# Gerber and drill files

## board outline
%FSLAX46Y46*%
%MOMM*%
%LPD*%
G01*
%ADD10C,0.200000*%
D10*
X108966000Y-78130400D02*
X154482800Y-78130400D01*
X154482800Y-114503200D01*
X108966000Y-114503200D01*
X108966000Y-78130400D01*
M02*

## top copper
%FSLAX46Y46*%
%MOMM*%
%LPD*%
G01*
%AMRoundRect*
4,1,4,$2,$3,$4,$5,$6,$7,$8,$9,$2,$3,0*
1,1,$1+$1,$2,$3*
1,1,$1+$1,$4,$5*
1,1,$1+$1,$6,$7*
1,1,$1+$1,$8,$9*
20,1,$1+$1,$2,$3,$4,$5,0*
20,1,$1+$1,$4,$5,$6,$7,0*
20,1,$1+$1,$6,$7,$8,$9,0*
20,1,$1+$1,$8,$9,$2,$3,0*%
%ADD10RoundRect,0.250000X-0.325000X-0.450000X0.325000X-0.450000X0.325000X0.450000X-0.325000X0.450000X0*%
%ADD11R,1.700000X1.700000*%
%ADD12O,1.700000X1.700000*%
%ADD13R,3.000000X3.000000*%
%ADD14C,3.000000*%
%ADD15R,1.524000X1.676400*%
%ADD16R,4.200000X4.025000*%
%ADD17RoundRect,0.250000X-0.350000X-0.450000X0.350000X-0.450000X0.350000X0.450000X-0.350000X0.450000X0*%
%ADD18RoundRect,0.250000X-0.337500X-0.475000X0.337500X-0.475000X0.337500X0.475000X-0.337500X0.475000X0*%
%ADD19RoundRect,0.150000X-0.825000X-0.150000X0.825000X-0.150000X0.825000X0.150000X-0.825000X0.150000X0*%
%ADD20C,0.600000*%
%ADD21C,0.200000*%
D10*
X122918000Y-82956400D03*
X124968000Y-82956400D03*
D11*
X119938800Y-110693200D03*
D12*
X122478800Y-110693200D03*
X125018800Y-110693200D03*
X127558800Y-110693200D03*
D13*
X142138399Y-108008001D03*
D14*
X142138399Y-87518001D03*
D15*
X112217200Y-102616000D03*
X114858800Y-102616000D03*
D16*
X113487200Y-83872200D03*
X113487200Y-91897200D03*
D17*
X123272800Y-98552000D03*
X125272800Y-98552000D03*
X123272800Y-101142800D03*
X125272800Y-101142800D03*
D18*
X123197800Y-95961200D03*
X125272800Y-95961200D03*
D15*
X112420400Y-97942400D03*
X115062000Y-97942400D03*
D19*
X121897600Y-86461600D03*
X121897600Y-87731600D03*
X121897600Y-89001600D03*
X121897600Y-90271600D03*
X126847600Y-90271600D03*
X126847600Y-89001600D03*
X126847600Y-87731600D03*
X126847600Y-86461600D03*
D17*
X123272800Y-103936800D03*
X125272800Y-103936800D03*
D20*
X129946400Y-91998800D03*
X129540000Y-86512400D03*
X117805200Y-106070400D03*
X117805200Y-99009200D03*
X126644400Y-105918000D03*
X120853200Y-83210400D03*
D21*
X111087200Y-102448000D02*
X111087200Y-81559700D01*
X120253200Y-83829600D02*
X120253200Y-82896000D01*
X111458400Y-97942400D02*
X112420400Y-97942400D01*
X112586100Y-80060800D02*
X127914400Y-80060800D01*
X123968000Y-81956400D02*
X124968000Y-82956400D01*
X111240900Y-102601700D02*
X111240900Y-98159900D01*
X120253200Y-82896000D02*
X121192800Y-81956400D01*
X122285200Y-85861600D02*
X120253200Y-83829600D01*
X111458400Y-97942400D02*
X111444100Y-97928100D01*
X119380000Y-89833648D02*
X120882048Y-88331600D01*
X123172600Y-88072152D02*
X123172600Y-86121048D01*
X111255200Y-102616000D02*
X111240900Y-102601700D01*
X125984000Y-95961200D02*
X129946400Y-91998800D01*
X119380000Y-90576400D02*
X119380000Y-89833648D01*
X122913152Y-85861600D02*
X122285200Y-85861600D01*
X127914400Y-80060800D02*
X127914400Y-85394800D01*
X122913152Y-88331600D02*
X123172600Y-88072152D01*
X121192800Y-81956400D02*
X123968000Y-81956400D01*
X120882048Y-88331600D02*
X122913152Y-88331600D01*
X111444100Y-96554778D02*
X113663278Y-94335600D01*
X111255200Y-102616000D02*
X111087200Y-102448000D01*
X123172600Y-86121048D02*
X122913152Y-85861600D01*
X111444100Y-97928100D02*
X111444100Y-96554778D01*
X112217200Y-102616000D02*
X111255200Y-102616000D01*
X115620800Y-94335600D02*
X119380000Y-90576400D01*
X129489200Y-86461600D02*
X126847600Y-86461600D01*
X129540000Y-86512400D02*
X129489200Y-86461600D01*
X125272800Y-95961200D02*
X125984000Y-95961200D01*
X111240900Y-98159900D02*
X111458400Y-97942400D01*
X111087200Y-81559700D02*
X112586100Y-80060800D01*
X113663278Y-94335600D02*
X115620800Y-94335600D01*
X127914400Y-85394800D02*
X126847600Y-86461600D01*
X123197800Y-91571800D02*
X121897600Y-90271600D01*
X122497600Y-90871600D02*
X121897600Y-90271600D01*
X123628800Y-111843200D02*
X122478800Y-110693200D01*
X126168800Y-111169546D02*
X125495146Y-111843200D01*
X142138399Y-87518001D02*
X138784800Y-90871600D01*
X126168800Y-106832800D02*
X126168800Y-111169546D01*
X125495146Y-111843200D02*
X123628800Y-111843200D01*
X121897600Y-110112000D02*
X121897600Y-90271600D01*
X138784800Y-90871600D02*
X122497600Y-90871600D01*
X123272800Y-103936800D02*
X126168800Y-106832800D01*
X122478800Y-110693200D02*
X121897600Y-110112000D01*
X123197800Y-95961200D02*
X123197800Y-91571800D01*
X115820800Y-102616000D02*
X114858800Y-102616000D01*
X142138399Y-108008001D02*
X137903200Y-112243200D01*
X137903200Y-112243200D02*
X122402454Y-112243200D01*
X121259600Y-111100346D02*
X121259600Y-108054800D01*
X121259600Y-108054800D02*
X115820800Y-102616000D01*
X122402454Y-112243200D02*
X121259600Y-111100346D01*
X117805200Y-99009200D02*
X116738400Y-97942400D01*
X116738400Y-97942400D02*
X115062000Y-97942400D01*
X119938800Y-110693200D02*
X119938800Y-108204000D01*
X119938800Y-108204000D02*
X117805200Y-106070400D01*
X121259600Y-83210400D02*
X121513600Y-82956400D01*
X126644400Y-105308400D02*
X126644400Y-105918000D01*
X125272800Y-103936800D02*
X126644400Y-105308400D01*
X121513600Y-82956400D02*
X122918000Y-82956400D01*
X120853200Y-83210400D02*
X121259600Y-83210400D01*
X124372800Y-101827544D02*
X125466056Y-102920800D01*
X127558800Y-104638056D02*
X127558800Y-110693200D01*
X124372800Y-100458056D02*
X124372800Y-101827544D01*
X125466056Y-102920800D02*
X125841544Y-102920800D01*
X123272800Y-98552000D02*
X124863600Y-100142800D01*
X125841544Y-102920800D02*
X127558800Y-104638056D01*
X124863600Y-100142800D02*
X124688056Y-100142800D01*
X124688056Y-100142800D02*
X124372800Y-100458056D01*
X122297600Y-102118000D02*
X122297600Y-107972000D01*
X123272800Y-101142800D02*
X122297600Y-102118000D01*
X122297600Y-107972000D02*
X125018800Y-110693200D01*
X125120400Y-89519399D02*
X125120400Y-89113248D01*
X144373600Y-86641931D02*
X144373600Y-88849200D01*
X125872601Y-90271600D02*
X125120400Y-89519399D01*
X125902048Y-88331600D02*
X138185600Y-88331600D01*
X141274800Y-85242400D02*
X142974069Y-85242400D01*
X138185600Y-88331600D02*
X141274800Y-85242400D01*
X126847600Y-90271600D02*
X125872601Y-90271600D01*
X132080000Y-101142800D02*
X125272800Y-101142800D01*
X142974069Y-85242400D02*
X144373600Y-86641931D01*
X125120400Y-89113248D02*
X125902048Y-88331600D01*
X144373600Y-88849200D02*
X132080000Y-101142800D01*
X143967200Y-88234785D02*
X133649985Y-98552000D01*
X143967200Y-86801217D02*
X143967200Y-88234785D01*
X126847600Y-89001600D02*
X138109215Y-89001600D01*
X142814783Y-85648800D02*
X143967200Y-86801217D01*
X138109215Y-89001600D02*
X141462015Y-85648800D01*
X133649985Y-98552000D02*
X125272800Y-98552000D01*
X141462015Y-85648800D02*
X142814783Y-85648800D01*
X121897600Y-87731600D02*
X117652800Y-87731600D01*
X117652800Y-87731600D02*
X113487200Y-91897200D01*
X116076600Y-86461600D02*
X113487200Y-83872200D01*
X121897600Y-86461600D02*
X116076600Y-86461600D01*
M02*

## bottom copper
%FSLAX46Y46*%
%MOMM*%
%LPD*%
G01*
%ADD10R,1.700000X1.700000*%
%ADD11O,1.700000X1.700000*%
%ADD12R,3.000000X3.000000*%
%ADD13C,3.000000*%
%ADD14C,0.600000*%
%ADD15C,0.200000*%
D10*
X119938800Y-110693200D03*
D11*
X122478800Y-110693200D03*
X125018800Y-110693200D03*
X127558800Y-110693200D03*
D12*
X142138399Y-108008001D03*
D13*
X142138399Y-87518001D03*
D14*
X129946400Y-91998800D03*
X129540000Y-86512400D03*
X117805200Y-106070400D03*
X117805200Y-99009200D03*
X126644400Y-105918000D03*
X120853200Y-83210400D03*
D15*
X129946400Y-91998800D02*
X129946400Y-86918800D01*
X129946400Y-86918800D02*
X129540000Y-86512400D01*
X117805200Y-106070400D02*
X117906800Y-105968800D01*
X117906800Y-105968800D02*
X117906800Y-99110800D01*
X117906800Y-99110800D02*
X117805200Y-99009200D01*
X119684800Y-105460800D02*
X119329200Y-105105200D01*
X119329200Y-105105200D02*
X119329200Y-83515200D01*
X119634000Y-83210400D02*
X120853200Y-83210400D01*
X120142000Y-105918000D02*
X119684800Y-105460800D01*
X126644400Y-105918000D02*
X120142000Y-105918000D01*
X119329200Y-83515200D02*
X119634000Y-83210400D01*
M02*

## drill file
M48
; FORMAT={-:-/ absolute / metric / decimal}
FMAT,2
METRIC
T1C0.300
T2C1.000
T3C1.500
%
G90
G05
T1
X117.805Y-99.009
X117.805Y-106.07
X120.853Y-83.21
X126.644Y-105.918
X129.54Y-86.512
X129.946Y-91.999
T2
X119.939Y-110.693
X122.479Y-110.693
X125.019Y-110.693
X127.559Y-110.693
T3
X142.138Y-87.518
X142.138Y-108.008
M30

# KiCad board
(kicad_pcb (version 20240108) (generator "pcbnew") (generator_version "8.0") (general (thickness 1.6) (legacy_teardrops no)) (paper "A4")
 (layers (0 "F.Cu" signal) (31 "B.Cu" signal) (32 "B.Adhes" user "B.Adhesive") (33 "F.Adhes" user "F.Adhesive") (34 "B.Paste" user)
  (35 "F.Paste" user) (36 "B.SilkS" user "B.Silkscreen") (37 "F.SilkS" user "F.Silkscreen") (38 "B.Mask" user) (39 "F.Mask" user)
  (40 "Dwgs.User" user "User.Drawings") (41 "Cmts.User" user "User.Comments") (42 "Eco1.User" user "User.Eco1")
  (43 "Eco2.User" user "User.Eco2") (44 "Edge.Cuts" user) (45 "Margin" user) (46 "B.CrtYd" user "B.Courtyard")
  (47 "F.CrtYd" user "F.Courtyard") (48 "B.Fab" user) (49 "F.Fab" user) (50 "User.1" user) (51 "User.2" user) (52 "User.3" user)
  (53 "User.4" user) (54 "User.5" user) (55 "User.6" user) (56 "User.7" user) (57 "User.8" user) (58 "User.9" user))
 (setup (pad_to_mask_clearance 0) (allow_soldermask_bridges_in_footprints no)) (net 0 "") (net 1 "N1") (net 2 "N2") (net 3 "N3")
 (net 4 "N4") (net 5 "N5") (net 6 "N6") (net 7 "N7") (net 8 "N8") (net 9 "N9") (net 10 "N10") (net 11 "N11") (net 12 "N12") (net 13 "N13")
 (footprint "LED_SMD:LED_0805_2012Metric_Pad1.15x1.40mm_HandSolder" (layer "F.Cu") (at 123.943 82.9564)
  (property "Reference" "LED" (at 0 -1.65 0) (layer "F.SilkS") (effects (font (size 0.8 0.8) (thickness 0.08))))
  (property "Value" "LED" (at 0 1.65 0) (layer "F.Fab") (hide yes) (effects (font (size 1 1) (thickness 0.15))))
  (pad "1" smd roundrect (at -1.025 0) (size 1.15 1.4) (layers "F.Cu" "F.Paste" "F.Mask") (roundrect_rratio 0.217391) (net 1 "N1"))
  (pad "2" smd roundrect (at 1.025 0) (size 1.15 1.4) (layers "F.Cu" "F.Paste" "F.Mask") (roundrect_rratio 0.217391) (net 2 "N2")))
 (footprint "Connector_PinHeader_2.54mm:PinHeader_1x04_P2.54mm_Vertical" (layer "F.Cu") (at 119.9388 110.6932 90)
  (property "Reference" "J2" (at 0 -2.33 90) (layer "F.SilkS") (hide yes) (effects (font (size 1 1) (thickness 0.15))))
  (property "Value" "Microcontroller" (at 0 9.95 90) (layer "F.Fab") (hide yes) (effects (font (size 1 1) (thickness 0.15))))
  (pad "1" thru_hole rect (at 0 0 90) (size 1.7 1.7) (drill 1) (layers "*.Cu" "*.Mask") (remove_unused_layers no) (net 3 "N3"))
  (pad "2" thru_hole oval (at 0 2.54 90) (size 1.7 1.7) (drill 1) (layers "*.Cu" "*.Mask") (remove_unused_layers no) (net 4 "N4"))
  (pad "3" thru_hole oval (at 0 5.08 90) (size 1.7 1.7) (drill 1) (layers "*.Cu" "*.Mask") (remove_unused_layers no) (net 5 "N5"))
  (pad "4" thru_hole oval (at 0 7.62 90) (size 1.7 1.7) (drill 1) (layers "*.Cu" "*.Mask") (remove_unused_layers no) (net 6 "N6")))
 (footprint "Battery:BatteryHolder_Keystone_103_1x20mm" (layer "F.Cu") (at 142.138399 108.008001 90)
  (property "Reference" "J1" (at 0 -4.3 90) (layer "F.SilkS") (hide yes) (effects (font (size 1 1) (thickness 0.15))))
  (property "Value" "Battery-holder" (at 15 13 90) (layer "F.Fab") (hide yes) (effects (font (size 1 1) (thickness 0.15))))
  (pad "1" thru_hole rect (at 0 0 90) (size 3 3) (drill 1.5) (layers "*.Cu" "*.Mask") (remove_unused_layers no) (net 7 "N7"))
  (pad "2" thru_hole circle (at 20.49 0 90) (size 3 3) (drill 1.5) (layers "*.Cu" "*.Mask") (remove_unused_layers no) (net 4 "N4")))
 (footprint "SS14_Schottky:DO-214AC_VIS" (layer "F.Cu") (at 113.538 102.616)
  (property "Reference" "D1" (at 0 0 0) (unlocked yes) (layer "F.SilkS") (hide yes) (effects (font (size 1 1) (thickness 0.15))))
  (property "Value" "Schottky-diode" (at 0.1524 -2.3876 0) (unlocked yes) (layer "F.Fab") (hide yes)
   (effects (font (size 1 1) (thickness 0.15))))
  (pad "1" smd rect (at -1.3208 0) (size 1.524 1.6764) (layers "F.Cu" "F.Paste" "F.Mask") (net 2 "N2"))
  (pad "2" smd rect (at 1.3208 0) (size 1.524 1.6764) (layers "F.Cu" "F.Paste" "F.Mask") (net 7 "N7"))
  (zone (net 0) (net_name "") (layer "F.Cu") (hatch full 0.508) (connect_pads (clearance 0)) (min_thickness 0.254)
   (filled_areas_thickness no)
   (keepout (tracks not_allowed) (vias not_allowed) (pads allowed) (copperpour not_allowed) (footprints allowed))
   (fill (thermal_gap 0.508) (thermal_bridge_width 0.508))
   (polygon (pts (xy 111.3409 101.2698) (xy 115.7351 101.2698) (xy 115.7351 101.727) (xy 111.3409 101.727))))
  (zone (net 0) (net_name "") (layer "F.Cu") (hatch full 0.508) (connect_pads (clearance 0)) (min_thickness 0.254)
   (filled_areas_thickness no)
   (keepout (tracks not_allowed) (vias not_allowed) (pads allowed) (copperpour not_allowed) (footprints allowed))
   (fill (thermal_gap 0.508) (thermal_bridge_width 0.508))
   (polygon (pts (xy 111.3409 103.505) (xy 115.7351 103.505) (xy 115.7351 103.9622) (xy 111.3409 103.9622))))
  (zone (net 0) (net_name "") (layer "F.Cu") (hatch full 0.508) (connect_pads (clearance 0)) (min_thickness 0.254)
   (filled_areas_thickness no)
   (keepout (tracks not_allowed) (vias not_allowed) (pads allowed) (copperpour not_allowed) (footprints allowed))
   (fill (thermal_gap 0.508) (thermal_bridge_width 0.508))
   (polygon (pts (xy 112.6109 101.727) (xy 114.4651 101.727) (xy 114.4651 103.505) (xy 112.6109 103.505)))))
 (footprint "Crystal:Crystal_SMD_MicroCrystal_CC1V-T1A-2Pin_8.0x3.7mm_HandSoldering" (layer "F.Cu") (at 113.4872 87.8847 -90)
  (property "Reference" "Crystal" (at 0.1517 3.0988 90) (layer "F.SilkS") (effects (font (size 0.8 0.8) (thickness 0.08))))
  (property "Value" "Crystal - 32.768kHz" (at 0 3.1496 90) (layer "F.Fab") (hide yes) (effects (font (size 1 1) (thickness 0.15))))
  (pad "1" smd rect (at -4.0125 0 270) (size 4.025 4.2) (layers "F.Cu" "F.Paste" "F.Mask") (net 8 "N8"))
  (pad "2" smd rect (at 4.0125 0 270) (size 4.025 4.2) (layers "F.Cu" "F.Paste" "F.Mask") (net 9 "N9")))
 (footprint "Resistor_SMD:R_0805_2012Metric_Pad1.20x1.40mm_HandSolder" (layer "F.Cu") (at 124.2728 98.552)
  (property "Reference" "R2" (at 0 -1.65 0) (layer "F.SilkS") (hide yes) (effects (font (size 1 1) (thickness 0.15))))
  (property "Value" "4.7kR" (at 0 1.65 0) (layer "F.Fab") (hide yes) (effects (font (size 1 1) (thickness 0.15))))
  (pad "1" smd roundrect (at -1 0) (size 1.2 1.4) (layers "F.Cu" "F.Paste" "F.Mask") (roundrect_rratio 0.208333) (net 6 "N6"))
  (pad "2" smd roundrect (at 1 0) (size 1.2 1.4) (layers "F.Cu" "F.Paste" "F.Mask") (roundrect_rratio 0.208333) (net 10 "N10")))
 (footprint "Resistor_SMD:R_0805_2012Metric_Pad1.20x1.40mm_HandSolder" (layer "F.Cu") (at 124.2728 101.1428)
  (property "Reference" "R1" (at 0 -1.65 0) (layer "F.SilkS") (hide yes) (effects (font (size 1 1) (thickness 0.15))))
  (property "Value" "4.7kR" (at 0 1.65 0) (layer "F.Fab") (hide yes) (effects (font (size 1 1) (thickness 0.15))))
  (pad "1" smd roundrect (at -1 0) (size 1.2 1.4) (layers "F.Cu" "F.Paste" "F.Mask") (roundrect_rratio 0.208333) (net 5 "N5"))
  (pad "2" smd roundrect (at 1 0) (size 1.2 1.4) (layers "F.Cu" "F.Paste" "F.Mask") (roundrect_rratio 0.208333) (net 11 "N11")))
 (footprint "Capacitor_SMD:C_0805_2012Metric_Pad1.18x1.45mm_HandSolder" (layer "F.Cu") (at 124.2353 95.9612)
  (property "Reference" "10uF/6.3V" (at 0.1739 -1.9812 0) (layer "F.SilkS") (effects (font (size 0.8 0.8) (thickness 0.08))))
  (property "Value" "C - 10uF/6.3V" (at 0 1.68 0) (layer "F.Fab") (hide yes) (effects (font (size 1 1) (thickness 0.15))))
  (pad "1" smd roundrect (at -1.0375 0) (size 1.175 1.45) (layers "F.Cu" "F.Paste" "F.Mask") (roundrect_rratio 0.212766) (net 4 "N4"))
  (pad "2" smd roundrect (at 1.0375 0) (size 1.175 1.45) (layers "F.Cu" "F.Paste" "F.Mask") (roundrect_rratio 0.212766) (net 2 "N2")))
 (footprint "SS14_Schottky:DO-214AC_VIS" (layer "F.Cu") (at 113.7412 97.9424)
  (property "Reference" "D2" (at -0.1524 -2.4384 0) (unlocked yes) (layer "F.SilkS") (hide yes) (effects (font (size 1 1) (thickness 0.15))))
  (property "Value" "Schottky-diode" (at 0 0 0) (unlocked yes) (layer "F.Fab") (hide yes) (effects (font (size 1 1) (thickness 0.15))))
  (pad "1" smd rect (at -1.3208 0) (size 1.524 1.6764) (layers "F.Cu" "F.Paste" "F.Mask") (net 2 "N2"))
  (pad "2" smd rect (at 1.3208 0) (size 1.524 1.6764) (layers "F.Cu" "F.Paste" "F.Mask") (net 3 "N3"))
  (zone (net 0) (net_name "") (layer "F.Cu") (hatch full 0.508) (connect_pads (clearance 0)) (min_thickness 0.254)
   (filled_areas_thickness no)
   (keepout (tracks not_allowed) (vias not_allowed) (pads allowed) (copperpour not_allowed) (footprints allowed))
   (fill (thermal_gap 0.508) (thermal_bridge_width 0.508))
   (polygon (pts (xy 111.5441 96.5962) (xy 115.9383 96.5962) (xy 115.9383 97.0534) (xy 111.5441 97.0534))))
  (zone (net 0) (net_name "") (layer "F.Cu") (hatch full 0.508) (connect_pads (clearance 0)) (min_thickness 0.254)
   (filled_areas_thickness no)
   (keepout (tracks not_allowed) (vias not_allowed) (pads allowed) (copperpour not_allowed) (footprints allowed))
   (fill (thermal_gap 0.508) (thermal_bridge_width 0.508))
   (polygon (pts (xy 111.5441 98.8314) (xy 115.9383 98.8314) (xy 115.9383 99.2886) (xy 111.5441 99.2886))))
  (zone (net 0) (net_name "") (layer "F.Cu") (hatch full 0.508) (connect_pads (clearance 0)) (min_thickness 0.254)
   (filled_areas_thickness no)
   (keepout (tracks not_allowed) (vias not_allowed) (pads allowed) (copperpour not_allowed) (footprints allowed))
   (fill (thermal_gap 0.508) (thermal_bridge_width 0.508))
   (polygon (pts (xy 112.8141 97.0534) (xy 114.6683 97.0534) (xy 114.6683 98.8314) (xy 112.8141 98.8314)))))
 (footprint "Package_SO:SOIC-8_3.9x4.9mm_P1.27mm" (layer "F.Cu") (at 124.3726 88.3666)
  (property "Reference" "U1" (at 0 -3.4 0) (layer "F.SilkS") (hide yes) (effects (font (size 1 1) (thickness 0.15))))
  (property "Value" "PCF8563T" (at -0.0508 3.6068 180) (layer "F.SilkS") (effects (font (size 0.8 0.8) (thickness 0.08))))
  (pad "1" smd roundrect (at -2.475 -1.905) (size 1.95 0.6) (layers "F.Cu" "F.Paste" "F.Mask") (roundrect_rratio 0.25) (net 8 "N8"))
  (pad "2" smd roundrect (at -2.475 -0.635) (size 1.95 0.6) (layers "F.Cu" "F.Paste" "F.Mask") (roundrect_rratio 0.25) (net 9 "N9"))
  (pad "3" smd roundrect (at -2.475 0.635) (size 1.95 0.6) (layers "F.Cu" "F.Paste" "F.Mask") (roundrect_rratio 0.25) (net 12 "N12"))
  (pad "4" smd roundrect (at -2.475 1.905) (size 1.95 0.6) (layers "F.Cu" "F.Paste" "F.Mask") (roundrect_rratio 0.25) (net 4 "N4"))
  (pad "5" smd roundrect (at 2.475 1.905) (size 1.95 0.6) (layers "F.Cu" "F.Paste" "F.Mask") (roundrect_rratio 0.25) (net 11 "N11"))
  (pad "6" smd roundrect (at 2.475 0.635) (size 1.95 0.6) (layers "F.Cu" "F.Paste" "F.Mask") (roundrect_rratio 0.25) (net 10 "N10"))
  (pad "7" smd roundrect (at 2.475 -0.635) (size 1.95 0.6) (layers "F.Cu" "F.Paste" "F.Mask") (roundrect_rratio 0.25) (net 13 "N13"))
  (pad "8" smd roundrect (at 2.475 -1.905) (size 1.95 0.6) (layers "F.Cu" "F.Paste" "F.Mask") (roundrect_rratio 0.25) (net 2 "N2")))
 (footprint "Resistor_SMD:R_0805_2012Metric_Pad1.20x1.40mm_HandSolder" (layer "F.Cu") (at 124.2728 103.9368)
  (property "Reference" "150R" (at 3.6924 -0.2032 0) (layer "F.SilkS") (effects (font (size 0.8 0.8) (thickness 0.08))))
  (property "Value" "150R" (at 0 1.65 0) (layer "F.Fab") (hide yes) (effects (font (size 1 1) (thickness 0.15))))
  (pad "1" smd roundrect (at -1 0) (size 1.2 1.4) (layers "F.Cu" "F.Paste" "F.Mask") (roundrect_rratio 0.208333) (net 4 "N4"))
  (pad "2" smd roundrect (at 1 0) (size 1.2 1.4) (layers "F.Cu" "F.Paste" "F.Mask") (roundrect_rratio 0.208333) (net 1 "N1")))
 (gr_rect (start 108.966 78.1304) (end 154.4828 114.5032) (stroke (width 0.2) (type default)) (fill none) (layer "Edge.Cuts"))
 (segment (start 111.0872 102.448) (end 111.0872 81.5597) (width 0.2) (layer "F.Cu") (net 2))
 (segment (start 120.2532 83.8296) (end 120.2532 82.896) (width 0.2) (layer "F.Cu") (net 2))
 (segment (start 111.4584 97.9424) (end 112.4204 97.9424) (width 0.2) (layer "F.Cu") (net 2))
 (segment (start 112.5861 80.0608) (end 127.9144 80.0608) (width 0.2) (layer "F.Cu") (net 2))
 (segment (start 123.968 81.9564) (end 124.968 82.9564) (width 0.2) (layer "F.Cu") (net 2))
 (segment (start 111.2409 102.6017) (end 111.2409 98.1599) (width 0.2) (layer "F.Cu") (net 2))
 (segment (start 120.2532 82.896) (end 121.1928 81.9564) (width 0.2) (layer "F.Cu") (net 2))
 (segment (start 122.2852 85.8616) (end 120.2532 83.8296) (width 0.2) (layer "F.Cu") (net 2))
 (segment (start 111.4584 97.9424) (end 111.4441 97.9281) (width 0.2) (layer "F.Cu") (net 2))
 (segment (start 119.38 89.833648) (end 120.882048 88.3316) (width 0.2) (layer "F.Cu") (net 2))
 (segment (start 123.1726 88.072152) (end 123.1726 86.121048) (width 0.2) (layer "F.Cu") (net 2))
 (segment (start 111.2552 102.616) (end 111.2409 102.6017) (width 0.2) (layer "F.Cu") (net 2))
 (segment (start 125.984 95.9612) (end 129.9464 91.9988) (width 0.2) (layer "F.Cu") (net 2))
 (segment (start 119.38 90.5764) (end 119.38 89.833648) (width 0.2) (layer "F.Cu") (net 2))
 (segment (start 122.913152 85.8616) (end 122.2852 85.8616) (width 0.2) (layer "F.Cu") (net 2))
 (segment (start 127.9144 80.0608) (end 127.9144 85.3948) (width 0.2) (layer "F.Cu") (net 2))
 (segment (start 122.913152 88.3316) (end 123.1726 88.072152) (width 0.2) (layer "F.Cu") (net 2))
 (segment (start 121.1928 81.9564) (end 123.968 81.9564) (width 0.2) (layer "F.Cu") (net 2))
 (segment (start 120.882048 88.3316) (end 122.913152 88.3316) (width 0.2) (layer "F.Cu") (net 2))
 (segment (start 111.4441 96.554778) (end 113.663278 94.3356) (width 0.2) (layer "F.Cu") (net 2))
 (segment (start 111.2552 102.616) (end 111.0872 102.448) (width 0.2) (layer "F.Cu") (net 2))
 (segment (start 123.1726 86.121048) (end 122.913152 85.8616) (width 0.2) (layer "F.Cu") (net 2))
 (segment (start 111.4441 97.9281) (end 111.4441 96.554778) (width 0.2) (layer "F.Cu") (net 2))
 (segment (start 112.2172 102.616) (end 111.2552 102.616) (width 0.2) (layer "F.Cu") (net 2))
 (segment (start 115.6208 94.3356) (end 119.38 90.5764) (width 0.2) (layer "F.Cu") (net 2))
 (segment (start 129.4892 86.4616) (end 126.8476 86.4616) (width 0.2) (layer "F.Cu") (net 2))
 (segment (start 129.54 86.5124) (end 129.4892 86.4616) (width 0.2) (layer "F.Cu") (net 2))
 (segment (start 125.2728 95.9612) (end 125.984 95.9612) (width 0.2) (layer "F.Cu") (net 2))
 (segment (start 111.2409 98.1599) (end 111.4584 97.9424) (width 0.2) (layer "F.Cu") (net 2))
 (segment (start 111.0872 81.5597) (end 112.5861 80.0608) (width 0.2) (layer "F.Cu") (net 2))
 (segment (start 113.663278 94.3356) (end 115.6208 94.3356) (width 0.2) (layer "F.Cu") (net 2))
 (segment (start 127.9144 85.3948) (end 126.8476 86.4616) (width 0.2) (layer "F.Cu") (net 2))
 (via (at 129.9464 91.9988) (size 0.6) (drill 0.3) (layers "F.Cu" "B.Cu") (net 2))
 (via (at 129.54 86.5124) (size 0.6) (drill 0.3) (layers "F.Cu" "B.Cu") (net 2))
 (segment (start 129.9464 91.9988) (end 129.9464 86.9188) (width 0.2) (layer "B.Cu") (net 2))
 (segment (start 129.9464 86.9188) (end 129.54 86.5124) (width 0.2) (layer "B.Cu") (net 2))
 (segment (start 123.1978 91.5718) (end 121.8976 90.2716) (width 0.2) (layer "F.Cu") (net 4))
 (segment (start 122.4976 90.8716) (end 121.8976 90.2716) (width 0.2) (layer "F.Cu") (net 4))
 (segment (start 123.6288 111.8432) (end 122.4788 110.6932) (width 0.2) (layer "F.Cu") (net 4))
 (segment (start 126.1688 111.169546) (end 125.495146 111.8432) (width 0.2) (layer "F.Cu") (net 4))
 (segment (start 142.138399 87.518001) (end 138.7848 90.8716) (width 0.2) (layer "F.Cu") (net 4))
 (segment (start 126.1688 106.8328) (end 126.1688 111.169546) (width 0.2) (layer "F.Cu") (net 4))
 (segment (start 125.495146 111.8432) (end 123.6288 111.8432) (width 0.2) (layer "F.Cu") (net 4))
 (segment (start 121.8976 110.112) (end 121.8976 90.2716) (width 0.2) (layer "F.Cu") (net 4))
 (segment (start 138.7848 90.8716) (end 122.4976 90.8716) (width 0.2) (layer "F.Cu") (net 4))
 (segment (start 123.2728 103.9368) (end 126.1688 106.8328) (width 0.2) (layer "F.Cu") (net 4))
 (segment (start 122.4788 110.6932) (end 121.8976 110.112) (width 0.2) (layer "F.Cu") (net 4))
 (segment (start 123.1978 95.9612) (end 123.1978 91.5718) (width 0.2) (layer "F.Cu") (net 4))
 (segment (start 115.8208 102.616) (end 114.8588 102.616) (width 0.2) (layer "F.Cu") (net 7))
 (segment (start 142.138399 108.008001) (end 137.9032 112.2432) (width 0.2) (layer "F.Cu") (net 7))
 (segment (start 137.9032 112.2432) (end 122.402454 112.2432) (width 0.2) (layer "F.Cu") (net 7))
 (segment (start 121.2596 111.100346) (end 121.2596 108.0548) (width 0.2) (layer "F.Cu") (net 7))
 (segment (start 121.2596 108.0548) (end 115.8208 102.616) (width 0.2) (layer "F.Cu") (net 7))
 (segment (start 122.402454 112.2432) (end 121.2596 111.100346) (width 0.2) (layer "F.Cu") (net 7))
 (segment (start 117.8052 99.0092) (end 116.7384 97.9424) (width 0.2) (layer "F.Cu") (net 3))
 (segment (start 116.7384 97.9424) (end 115.062 97.9424) (width 0.2) (layer "F.Cu") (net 3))
 (segment (start 119.9388 110.6932) (end 119.9388 108.204) (width 0.2) (layer "F.Cu") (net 3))
 (segment (start 119.9388 108.204) (end 117.8052 106.0704) (width 0.2) (layer "F.Cu") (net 3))
 (via (at 117.8052 106.0704) (size 0.6) (drill 0.3) (layers "F.Cu" "B.Cu") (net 3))
 (via (at 117.8052 99.0092) (size 0.6) (drill 0.3) (layers "F.Cu" "B.Cu") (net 3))
 (segment (start 117.8052 106.0704) (end 117.9068 105.9688) (width 0.2) (layer "B.Cu") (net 3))
 (segment (start 117.9068 105.9688) (end 117.9068 99.1108) (width 0.2) (layer "B.Cu") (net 3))
 (segment (start 117.9068 99.1108) (end 117.8052 99.0092) (width 0.2) (layer "B.Cu") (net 3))
 (segment (start 121.2596 83.2104) (end 121.5136 82.9564) (width 0.2) (layer "F.Cu") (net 1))
 (segment (start 126.6444 105.3084) (end 126.6444 105.918) (width 0.2) (layer "F.Cu") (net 1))
 (segment (start 125.2728 103.9368) (end 126.6444 105.3084) (width 0.2) (layer "F.Cu") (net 1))
 (segment (start 121.5136 82.9564) (end 122.918 82.9564) (width 0.2) (layer "F.Cu") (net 1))
 (segment (start 120.8532 83.2104) (end 121.2596 83.2104) (width 0.2) (layer "F.Cu") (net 1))
 (via (at 126.6444 105.918) (size 0.6) (drill 0.3) (layers "F.Cu" "B.Cu") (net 1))
 (via (at 120.8532 83.2104) (size 0.6) (drill 0.3) (layers "F.Cu" "B.Cu") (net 1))
 (segment (start 119.6848 105.4608) (end 119.3292 105.1052) (width 0.2) (layer "B.Cu") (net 1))
 (segment (start 119.3292 105.1052) (end 119.3292 83.5152) (width 0.2) (layer "B.Cu") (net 1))
 (segment (start 119.634 83.2104) (end 120.8532 83.2104) (width 0.2) (layer "B.Cu") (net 1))
 (segment (start 120.142 105.918) (end 119.6848 105.4608) (width 0.2) (layer "B.Cu") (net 1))
 (segment (start 126.6444 105.918) (end 120.142 105.918) (width 0.2) (layer "B.Cu") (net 1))
 (segment (start 119.3292 83.5152) (end 119.634 83.2104) (width 0.2) (layer "B.Cu") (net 1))
 (segment (start 124.3728 101.827544) (end 125.466056 102.9208) (width 0.2) (layer "F.Cu") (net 6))
 (segment (start 127.5588 104.638056) (end 127.5588 110.6932) (width 0.2) (layer "F.Cu") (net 6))
 (segment (start 124.3728 100.458056) (end 124.3728 101.827544) (width 0.2) (layer "F.Cu") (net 6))
 (segment (start 125.466056 102.9208) (end 125.841544 102.9208) (width 0.2) (layer "F.Cu") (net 6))
 (segment (start 123.2728 98.552) (end 124.8636 100.1428) (width 0.2) (layer "F.Cu") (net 6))
 (segment (start 125.841544 102.9208) (end 127.5588 104.638056) (width 0.2) (layer "F.Cu") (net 6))
 (segment (start 124.8636 100.1428) (end 124.688056 100.1428) (width 0.2) (layer "F.Cu") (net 6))
 (segment (start 124.688056 100.1428) (end 124.3728 100.458056) (width 0.2) (layer "F.Cu") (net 6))
 (segment (start 122.2976 102.118) (end 122.2976 107.972) (width 0.2) (layer "F.Cu") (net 5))
 (segment (start 123.2728 101.1428) (end 122.2976 102.118) (width 0.2) (layer "F.Cu") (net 5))
 (segment (start 122.2976 107.972) (end 125.0188 110.6932) (width 0.2) (layer "F.Cu") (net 5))
 (segment (start 125.1204 89.519399) (end 125.1204 89.113248) (width 0.2) (layer "F.Cu") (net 11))
 (segment (start 144.3736 86.641931) (end 144.3736 88.8492) (width 0.2) (layer "F.Cu") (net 11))
 (segment (start 125.872601 90.2716) (end 125.1204 89.519399) (width 0.2) (layer "F.Cu") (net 11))
 (segment (start 125.902048 88.3316) (end 138.1856 88.3316) (width 0.2) (layer "F.Cu") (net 11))
 (segment (start 141.2748 85.2424) (end 142.974069 85.2424) (width 0.2) (layer "F.Cu") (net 11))
 (segment (start 138.1856 88.3316) (end 141.2748 85.2424) (width 0.2) (layer "F.Cu") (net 11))
 (segment (start 126.8476 90.2716) (end 125.872601 90.2716) (width 0.2) (layer "F.Cu") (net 11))
 (segment (start 132.08 101.1428) (end 125.2728 101.1428) (width 0.2) (layer "F.Cu") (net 11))
 (segment (start 142.974069 85.2424) (end 144.3736 86.641931) (width 0.2) (layer "F.Cu") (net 11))
 (segment (start 125.1204 89.113248) (end 125.902048 88.3316) (width 0.2) (layer "F.Cu") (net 11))
 (segment (start 144.3736 88.8492) (end 132.08 101.1428) (width 0.2) (layer "F.Cu") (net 11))
 (segment (start 143.9672 88.234785) (end 133.649985 98.552) (width 0.2) (layer "F.Cu") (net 10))
 (segment (start 143.9672 86.801217) (end 143.9672 88.234785) (width 0.2) (layer "F.Cu") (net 10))
 (segment (start 126.8476 89.0016) (end 138.109215 89.0016) (width 0.2) (layer "F.Cu") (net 10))
 (segment (start 142.814783 85.6488) (end 143.9672 86.801217) (width 0.2) (layer "F.Cu") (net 10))
 (segment (start 138.109215 89.0016) (end 141.462015 85.6488) (width 0.2) (layer "F.Cu") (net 10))
 (segment (start 133.649985 98.552) (end 125.2728 98.552) (width 0.2) (layer "F.Cu") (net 10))
 (segment (start 141.462015 85.6488) (end 142.814783 85.6488) (width 0.2) (layer "F.Cu") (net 10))
 (segment (start 121.8976 87.7316) (end 117.6528 87.7316) (width 0.2) (layer "F.Cu") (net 9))
 (segment (start 117.6528 87.7316) (end 113.4872 91.8972) (width 0.2) (layer "F.Cu") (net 9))
 (segment (start 116.0766 86.4616) (end 113.4872 83.8722) (width 0.2) (layer "F.Cu") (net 8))
 (segment (start 121.8976 86.4616) (end 116.0766 86.4616) (width 0.2) (layer "F.Cu") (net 8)))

